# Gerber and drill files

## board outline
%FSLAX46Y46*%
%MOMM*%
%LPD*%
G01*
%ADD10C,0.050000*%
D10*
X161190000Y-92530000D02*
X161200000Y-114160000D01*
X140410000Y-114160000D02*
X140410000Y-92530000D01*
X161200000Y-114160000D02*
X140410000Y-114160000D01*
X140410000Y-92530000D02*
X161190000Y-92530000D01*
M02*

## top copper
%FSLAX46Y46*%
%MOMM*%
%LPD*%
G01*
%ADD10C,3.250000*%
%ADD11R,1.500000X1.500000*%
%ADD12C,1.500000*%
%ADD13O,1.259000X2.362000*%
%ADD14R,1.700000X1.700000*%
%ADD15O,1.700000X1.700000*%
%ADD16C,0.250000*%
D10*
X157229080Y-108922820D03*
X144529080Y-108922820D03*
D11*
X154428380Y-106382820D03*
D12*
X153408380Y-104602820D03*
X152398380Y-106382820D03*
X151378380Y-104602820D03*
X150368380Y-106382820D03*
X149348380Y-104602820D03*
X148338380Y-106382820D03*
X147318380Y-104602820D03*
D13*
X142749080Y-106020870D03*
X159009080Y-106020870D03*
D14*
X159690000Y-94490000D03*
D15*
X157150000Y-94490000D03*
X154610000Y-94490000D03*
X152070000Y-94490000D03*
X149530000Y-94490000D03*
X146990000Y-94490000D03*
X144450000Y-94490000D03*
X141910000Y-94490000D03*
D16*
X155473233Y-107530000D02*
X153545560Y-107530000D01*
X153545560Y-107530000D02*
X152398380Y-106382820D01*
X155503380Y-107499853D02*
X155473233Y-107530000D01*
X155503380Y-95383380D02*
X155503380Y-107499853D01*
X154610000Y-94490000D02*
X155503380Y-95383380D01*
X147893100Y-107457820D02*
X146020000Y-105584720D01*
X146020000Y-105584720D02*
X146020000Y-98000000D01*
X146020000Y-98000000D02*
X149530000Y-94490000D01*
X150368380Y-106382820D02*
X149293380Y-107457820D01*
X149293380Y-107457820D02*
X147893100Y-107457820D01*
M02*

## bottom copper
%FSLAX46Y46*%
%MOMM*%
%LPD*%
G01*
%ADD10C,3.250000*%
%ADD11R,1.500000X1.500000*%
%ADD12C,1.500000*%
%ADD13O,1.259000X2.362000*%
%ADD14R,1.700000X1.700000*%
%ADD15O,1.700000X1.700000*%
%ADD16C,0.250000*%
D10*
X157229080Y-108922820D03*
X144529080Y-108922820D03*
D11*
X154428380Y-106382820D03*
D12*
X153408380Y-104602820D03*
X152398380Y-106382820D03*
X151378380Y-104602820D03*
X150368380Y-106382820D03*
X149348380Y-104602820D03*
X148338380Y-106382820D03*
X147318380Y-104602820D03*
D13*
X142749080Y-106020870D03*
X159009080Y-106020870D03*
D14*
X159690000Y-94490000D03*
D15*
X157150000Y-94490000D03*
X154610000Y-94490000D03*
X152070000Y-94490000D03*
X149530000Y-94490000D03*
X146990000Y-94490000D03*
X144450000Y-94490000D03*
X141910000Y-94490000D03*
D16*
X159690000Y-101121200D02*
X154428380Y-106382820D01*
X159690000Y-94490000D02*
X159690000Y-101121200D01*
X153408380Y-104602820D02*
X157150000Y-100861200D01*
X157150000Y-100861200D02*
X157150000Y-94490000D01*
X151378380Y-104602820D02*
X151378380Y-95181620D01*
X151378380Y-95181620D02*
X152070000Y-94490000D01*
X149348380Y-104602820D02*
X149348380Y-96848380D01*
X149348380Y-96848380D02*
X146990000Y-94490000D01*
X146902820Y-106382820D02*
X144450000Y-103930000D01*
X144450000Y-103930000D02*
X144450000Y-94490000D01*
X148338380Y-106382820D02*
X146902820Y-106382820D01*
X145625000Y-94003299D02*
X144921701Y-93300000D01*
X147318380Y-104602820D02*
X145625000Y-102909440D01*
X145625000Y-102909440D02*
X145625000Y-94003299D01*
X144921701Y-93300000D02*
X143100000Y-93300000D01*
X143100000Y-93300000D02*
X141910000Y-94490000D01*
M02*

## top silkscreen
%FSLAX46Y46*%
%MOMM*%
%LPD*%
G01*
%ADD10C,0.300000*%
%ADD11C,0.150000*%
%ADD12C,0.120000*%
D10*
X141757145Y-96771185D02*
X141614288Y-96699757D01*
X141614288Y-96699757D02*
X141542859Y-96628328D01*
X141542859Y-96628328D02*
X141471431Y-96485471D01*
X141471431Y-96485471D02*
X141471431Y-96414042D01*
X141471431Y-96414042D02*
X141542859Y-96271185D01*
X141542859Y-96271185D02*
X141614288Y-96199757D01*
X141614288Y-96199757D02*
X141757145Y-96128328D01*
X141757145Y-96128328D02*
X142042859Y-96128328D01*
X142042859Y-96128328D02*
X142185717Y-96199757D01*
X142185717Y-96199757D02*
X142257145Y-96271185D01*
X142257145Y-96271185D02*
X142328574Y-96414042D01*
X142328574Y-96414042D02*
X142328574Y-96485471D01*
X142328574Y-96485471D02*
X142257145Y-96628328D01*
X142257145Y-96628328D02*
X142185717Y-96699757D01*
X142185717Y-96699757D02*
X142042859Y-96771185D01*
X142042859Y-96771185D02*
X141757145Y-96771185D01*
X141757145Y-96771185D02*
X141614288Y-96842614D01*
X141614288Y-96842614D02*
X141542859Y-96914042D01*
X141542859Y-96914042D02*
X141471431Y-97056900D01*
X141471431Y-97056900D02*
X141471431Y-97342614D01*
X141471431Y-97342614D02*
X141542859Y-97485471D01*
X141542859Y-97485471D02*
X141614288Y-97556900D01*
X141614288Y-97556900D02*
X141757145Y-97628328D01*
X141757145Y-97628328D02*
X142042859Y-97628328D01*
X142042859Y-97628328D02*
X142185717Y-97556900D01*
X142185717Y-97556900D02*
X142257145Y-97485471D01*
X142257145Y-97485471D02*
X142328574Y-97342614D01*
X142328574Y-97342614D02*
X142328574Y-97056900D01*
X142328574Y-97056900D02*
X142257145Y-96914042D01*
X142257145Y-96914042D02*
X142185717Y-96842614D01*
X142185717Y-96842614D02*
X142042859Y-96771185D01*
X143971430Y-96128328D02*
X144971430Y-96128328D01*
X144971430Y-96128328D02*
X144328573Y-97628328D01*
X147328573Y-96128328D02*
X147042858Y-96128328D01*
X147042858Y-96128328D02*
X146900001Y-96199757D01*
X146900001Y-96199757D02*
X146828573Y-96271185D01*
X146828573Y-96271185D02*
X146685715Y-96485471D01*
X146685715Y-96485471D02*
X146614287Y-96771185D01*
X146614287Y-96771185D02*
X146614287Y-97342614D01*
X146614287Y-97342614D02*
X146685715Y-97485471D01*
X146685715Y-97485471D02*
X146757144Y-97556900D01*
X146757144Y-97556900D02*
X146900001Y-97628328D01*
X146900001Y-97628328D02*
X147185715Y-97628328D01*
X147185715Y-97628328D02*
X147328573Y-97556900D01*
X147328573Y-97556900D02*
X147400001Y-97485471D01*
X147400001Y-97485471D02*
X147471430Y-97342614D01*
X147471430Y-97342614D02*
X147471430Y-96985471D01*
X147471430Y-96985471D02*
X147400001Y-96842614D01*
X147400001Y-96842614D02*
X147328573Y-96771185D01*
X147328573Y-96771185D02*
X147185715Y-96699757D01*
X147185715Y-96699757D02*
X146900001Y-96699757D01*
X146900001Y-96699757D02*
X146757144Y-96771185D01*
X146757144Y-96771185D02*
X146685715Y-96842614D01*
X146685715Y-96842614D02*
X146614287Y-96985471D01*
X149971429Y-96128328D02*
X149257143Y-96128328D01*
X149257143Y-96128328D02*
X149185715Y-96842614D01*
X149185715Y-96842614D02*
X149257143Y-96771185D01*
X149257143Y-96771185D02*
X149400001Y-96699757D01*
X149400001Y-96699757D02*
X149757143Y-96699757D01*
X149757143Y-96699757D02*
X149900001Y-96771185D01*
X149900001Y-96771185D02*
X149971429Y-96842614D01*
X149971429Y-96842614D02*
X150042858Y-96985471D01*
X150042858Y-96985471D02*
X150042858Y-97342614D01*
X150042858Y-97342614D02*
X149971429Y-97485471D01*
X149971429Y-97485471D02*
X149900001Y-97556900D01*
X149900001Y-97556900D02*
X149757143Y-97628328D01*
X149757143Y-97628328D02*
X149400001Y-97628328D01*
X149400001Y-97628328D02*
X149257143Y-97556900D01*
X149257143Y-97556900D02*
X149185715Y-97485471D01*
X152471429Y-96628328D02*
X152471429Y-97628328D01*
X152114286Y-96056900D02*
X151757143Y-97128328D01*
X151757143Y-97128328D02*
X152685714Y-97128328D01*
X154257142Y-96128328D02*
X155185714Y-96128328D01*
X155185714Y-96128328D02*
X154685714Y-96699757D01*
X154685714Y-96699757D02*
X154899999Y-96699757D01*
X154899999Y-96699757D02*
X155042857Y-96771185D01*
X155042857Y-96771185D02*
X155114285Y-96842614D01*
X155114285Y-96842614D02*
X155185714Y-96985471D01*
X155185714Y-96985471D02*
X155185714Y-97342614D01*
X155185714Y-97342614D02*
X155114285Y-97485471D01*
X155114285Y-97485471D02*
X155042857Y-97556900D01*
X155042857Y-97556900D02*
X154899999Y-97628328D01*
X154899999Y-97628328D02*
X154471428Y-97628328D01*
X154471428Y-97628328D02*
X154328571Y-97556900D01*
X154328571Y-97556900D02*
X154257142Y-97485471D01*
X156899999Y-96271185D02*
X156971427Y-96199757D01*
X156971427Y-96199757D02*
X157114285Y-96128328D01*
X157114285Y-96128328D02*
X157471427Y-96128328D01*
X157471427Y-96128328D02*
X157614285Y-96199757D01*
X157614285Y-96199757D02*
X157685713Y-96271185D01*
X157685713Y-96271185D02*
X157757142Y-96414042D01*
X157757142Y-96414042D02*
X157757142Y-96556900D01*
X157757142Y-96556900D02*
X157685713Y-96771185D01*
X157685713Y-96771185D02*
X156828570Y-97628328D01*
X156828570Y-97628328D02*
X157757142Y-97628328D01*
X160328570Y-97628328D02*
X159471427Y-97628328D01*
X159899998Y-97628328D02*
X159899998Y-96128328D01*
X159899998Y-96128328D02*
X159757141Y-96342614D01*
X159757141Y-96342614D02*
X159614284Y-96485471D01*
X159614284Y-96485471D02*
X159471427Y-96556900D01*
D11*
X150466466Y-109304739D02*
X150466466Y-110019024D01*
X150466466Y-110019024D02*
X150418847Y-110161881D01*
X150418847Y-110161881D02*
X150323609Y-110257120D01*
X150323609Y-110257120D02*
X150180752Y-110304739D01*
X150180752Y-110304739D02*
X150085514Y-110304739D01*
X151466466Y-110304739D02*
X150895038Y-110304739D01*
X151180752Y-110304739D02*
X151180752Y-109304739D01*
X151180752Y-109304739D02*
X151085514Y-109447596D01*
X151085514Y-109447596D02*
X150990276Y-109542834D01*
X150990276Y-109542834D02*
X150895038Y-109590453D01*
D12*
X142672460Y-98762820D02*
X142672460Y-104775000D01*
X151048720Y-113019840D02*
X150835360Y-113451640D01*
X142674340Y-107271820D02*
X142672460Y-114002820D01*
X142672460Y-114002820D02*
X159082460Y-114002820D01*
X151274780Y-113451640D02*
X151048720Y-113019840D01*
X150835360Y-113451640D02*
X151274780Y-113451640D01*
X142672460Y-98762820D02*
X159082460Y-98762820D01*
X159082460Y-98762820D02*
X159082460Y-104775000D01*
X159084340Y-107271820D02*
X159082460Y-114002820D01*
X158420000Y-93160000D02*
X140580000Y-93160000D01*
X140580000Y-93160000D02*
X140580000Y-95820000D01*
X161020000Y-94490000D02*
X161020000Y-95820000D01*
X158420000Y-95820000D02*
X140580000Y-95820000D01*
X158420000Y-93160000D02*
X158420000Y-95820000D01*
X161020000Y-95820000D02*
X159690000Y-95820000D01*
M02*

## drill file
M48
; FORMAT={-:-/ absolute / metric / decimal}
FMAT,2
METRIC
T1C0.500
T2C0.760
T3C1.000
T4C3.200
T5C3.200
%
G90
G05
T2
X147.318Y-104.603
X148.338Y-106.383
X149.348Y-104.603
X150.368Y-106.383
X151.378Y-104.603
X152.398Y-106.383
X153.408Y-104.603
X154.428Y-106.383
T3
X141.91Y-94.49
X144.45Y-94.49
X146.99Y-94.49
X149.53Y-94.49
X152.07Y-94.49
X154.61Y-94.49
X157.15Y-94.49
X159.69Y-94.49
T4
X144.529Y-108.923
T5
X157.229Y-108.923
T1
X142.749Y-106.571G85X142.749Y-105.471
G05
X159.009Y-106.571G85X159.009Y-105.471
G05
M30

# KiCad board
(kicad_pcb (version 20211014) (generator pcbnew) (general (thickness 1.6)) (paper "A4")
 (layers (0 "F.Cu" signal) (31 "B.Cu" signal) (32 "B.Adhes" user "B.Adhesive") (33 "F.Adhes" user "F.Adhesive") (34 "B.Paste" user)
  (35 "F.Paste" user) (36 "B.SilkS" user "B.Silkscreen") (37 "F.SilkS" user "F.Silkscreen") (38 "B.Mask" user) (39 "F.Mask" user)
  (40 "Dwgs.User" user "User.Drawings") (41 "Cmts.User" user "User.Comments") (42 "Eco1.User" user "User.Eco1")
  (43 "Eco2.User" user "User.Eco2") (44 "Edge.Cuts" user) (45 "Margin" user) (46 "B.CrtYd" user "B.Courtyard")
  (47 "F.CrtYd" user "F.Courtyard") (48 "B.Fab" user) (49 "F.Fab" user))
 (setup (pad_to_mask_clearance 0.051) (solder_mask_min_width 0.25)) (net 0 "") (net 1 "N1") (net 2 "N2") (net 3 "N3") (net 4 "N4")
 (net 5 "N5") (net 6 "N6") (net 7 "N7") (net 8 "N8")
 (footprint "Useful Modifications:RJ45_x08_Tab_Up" (layer "F.Cu") (at 150.6474 109.982)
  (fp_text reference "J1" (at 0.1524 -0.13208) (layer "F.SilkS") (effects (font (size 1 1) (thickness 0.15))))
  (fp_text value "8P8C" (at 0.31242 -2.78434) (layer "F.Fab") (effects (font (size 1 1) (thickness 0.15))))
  (fp_line (start -7.97494 -11.21918) (end -7.97494 -5.207) (layer "F.SilkS") (width 0.12))
  (fp_line (start 0.40132 3.03784) (end 0.18796 3.46964) (layer "F.SilkS") (width 0.12))
  (fp_line (start -7.97306 -2.71018) (end -7.97494 4.02082) (layer "F.SilkS") (width 0.12))
  (fp_line (start -7.97494 4.02082) (end 8.43506 4.02082) (layer "F.SilkS") (width 0.12))
  (fp_line (start 0.62738 3.46964) (end 0.40132 3.03784) (layer "F.SilkS") (width 0.12))
  (fp_line (start 0.18796 3.46964) (end 0.62738 3.46964) (layer "F.SilkS") (width 0.12))
  (fp_line (start -7.97494 -11.21918) (end 8.43506 -11.21918) (layer "F.SilkS") (width 0.12))
  (fp_line (start 8.43506 -11.21918) (end 8.43506 -5.207) (layer "F.SilkS") (width 0.12))
  (fp_line (start 8.43694 -2.71018) (end 8.43506 4.02082) (layer "F.SilkS") (width 0.12))
  (pad "" np_thru_hole circle locked (at 6.58168 -1.05918 180) (size 3.25 3.25) (drill 3.200001) (layers *.Cu *.Mask))
  (pad "" np_thru_hole circle locked (at -6.11832 -1.05918 180) (size 3.25 3.25) (drill 3.2) (layers *.Cu *.Mask))
  (pad "1" thru_hole rect locked (at 3.78098 -3.59918) (size 1.5 1.5) (drill 0.76) (layers *.Cu *.Mask) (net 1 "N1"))
  (pad "2" thru_hole circle locked (at 2.76098 -5.37918) (size 1.5 1.5) (drill 0.76) (layers *.Cu *.Mask) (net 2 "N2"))
  (pad "3" thru_hole circle locked (at 1.75098 -3.59918) (size 1.5 1.5) (drill 0.76) (layers *.Cu *.Mask) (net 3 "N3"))
  (pad "4" thru_hole circle locked (at 0.73098 -5.37918) (size 1.5 1.5) (drill 0.76) (layers *.Cu *.Mask) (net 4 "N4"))
  (pad "5" thru_hole circle locked (at -0.27902 -3.59918) (size 1.5 1.5) (drill 0.76) (layers *.Cu *.Mask) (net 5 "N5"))
  (pad "6" thru_hole circle locked (at -1.29902 -5.37918) (size 1.5 1.5) (drill 0.76) (layers *.Cu *.Mask) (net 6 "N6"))
  (pad "7" thru_hole circle locked (at -2.30902 -3.59918) (size 1.5 1.5) (drill 0.76) (layers *.Cu *.Mask) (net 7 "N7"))
  (pad "8" thru_hole circle locked (at -3.32902 -5.37918) (size 1.5 1.5) (drill 0.76) (layers *.Cu *.Mask) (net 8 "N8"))
  (pad "9" thru_hole oval locked (at -7.89832 -3.96113 180) (size 1.259 2.362) (drill oval 0.5 1.6) (layers *.Cu *.Mask))
  (pad "10" thru_hole oval locked (at 8.36168 -3.96113 180) (size 1.259 2.362) (drill oval 0.5 1.6) (layers *.Cu *.Mask)))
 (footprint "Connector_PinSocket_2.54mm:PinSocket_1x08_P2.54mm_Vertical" (layer "F.Cu") (at 159.69 94.49 -90)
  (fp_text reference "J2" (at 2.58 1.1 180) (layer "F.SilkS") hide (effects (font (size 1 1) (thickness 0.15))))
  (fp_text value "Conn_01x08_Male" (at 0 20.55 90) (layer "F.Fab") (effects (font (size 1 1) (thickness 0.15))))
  (fp_line (start -1.33 1.27) (end -1.33 19.11) (layer "F.SilkS") (width 0.12))
  (fp_line (start -1.33 19.11) (end 1.33 19.11) (layer "F.SilkS") (width 0.12))
  (fp_line (start 0 -1.33) (end 1.33 -1.33) (layer "F.SilkS") (width 0.12))
  (fp_line (start 1.33 1.27) (end 1.33 19.11) (layer "F.SilkS") (width 0.12))
  (fp_line (start -1.33 1.27) (end 1.33 1.27) (layer "F.SilkS") (width 0.12))
  (fp_line (start 1.33 -1.33) (end 1.33 0) (layer "F.SilkS") (width 0.12))
  (pad "1" thru_hole rect (at 0 0 270) (size 1.7 1.7) (drill 1) (layers *.Cu *.Mask) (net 1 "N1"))
  (pad "2" thru_hole oval (at 0 2.54 270) (size 1.7 1.7) (drill 1) (layers *.Cu *.Mask) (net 2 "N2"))
  (pad "3" thru_hole oval (at 0 5.08 270) (size 1.7 1.7) (drill 1) (layers *.Cu *.Mask) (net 3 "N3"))
  (pad "4" thru_hole oval (at 0 7.62 270) (size 1.7 1.7) (drill 1) (layers *.Cu *.Mask) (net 4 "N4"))
  (pad "5" thru_hole oval (at 0 10.16 270) (size 1.7 1.7) (drill 1) (layers *.Cu *.Mask) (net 5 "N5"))
  (pad "6" thru_hole oval (at 0 12.7 270) (size 1.7 1.7) (drill 1) (layers *.Cu *.Mask) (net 6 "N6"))
  (pad "7" thru_hole oval (at 0 15.24 270) (size 1.7 1.7) (drill 1) (layers *.Cu *.Mask) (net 7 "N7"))
  (pad "8" thru_hole oval (at 0 17.78 270) (size 1.7 1.7) (drill 1) (layers *.Cu *.Mask) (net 8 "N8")))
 (gr_line (start 161.19 92.53) (end 161.2 114.16) (layer "Edge.Cuts") (width 0.05))
 (gr_line (start 140.41 114.16) (end 140.41 92.53) (layer "Edge.Cuts") (width 0.05))
 (gr_line (start 161.2 114.16) (end 140.41 114.16) (layer "Edge.Cuts") (width 0.05))
 (gr_line (start 140.41 92.53) (end 161.19 92.53) (layer "Edge.Cuts") (width 0.05))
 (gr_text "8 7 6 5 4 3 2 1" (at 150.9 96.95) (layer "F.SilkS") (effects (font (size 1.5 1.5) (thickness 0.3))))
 (segment (start 159.69 101.1212) (end 154.42838 106.38282) (width 0.25) (layer "B.Cu") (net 1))
 (segment (start 159.69 94.49) (end 159.69 101.1212) (width 0.25) (layer "B.Cu") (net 1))
 (segment (start 153.40838 104.60282) (end 157.15 100.8612) (width 0.25) (layer "B.Cu") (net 2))
 (segment (start 157.15 100.8612) (end 157.15 94.49) (width 0.25) (layer "B.Cu") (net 2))
 (segment (start 155.473233 107.53) (end 153.54556 107.53) (width 0.25) (layer "F.Cu") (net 3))
 (segment (start 153.54556 107.53) (end 152.39838 106.38282) (width 0.25) (layer "F.Cu") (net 3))
 (segment (start 155.50338 107.499853) (end 155.473233 107.53) (width 0.25) (layer "F.Cu") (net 3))
 (segment (start 155.50338 95.38338) (end 155.50338 107.499853) (width 0.25) (layer "F.Cu") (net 3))
 (segment (start 154.61 94.49) (end 155.50338 95.38338) (width 0.25) (layer "F.Cu") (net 3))
 (segment (start 151.37838 104.60282) (end 151.37838 95.18162) (width 0.25) (layer "B.Cu") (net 4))
 (segment (start 151.37838 95.18162) (end 152.07 94.49) (width 0.25) (layer "B.Cu") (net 4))
 (segment (start 147.8931 107.45782) (end 146.02 105.58472) (width 0.25) (layer "F.Cu") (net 5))
 (segment (start 146.02 105.58472) (end 146.02 98) (width 0.25) (layer "F.Cu") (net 5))
 (segment (start 146.02 98) (end 149.53 94.49) (width 0.25) (layer "F.Cu") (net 5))
 (segment (start 150.36838 106.38282) (end 149.29338 107.45782) (width 0.25) (layer "F.Cu") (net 5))
 (segment (start 149.29338 107.45782) (end 147.8931 107.45782) (width 0.25) (layer "F.Cu") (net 5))
 (segment (start 149.34838 104.60282) (end 149.34838 96.84838) (width 0.25) (layer "B.Cu") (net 6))
 (segment (start 149.34838 96.84838) (end 146.99 94.49) (width 0.25) (layer "B.Cu") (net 6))
 (segment (start 146.90282 106.38282) (end 144.45 103.93) (width 0.25) (layer "B.Cu") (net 7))
 (segment (start 144.45 103.93) (end 144.45 94.49) (width 0.25) (layer "B.Cu") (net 7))
 (segment (start 148.33838 106.38282) (end 146.90282 106.38282) (width 0.25) (layer "B.Cu") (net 7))
 (segment (start 145.625 94.003299) (end 144.921701 93.3) (width 0.25) (layer "B.Cu") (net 8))
 (segment (start 147.31838 104.60282) (end 145.625 102.90944) (width 0.25) (layer "B.Cu") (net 8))
 (segment (start 145.625 102.90944) (end 145.625 94.003299) (width 0.25) (layer "B.Cu") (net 8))
 (segment (start 144.921701 93.3) (end 143.1 93.3) (width 0.25) (layer "B.Cu") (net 8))
 (segment (start 143.1 93.3) (end 141.91 94.49) (width 0.25) (layer "B.Cu") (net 8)))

